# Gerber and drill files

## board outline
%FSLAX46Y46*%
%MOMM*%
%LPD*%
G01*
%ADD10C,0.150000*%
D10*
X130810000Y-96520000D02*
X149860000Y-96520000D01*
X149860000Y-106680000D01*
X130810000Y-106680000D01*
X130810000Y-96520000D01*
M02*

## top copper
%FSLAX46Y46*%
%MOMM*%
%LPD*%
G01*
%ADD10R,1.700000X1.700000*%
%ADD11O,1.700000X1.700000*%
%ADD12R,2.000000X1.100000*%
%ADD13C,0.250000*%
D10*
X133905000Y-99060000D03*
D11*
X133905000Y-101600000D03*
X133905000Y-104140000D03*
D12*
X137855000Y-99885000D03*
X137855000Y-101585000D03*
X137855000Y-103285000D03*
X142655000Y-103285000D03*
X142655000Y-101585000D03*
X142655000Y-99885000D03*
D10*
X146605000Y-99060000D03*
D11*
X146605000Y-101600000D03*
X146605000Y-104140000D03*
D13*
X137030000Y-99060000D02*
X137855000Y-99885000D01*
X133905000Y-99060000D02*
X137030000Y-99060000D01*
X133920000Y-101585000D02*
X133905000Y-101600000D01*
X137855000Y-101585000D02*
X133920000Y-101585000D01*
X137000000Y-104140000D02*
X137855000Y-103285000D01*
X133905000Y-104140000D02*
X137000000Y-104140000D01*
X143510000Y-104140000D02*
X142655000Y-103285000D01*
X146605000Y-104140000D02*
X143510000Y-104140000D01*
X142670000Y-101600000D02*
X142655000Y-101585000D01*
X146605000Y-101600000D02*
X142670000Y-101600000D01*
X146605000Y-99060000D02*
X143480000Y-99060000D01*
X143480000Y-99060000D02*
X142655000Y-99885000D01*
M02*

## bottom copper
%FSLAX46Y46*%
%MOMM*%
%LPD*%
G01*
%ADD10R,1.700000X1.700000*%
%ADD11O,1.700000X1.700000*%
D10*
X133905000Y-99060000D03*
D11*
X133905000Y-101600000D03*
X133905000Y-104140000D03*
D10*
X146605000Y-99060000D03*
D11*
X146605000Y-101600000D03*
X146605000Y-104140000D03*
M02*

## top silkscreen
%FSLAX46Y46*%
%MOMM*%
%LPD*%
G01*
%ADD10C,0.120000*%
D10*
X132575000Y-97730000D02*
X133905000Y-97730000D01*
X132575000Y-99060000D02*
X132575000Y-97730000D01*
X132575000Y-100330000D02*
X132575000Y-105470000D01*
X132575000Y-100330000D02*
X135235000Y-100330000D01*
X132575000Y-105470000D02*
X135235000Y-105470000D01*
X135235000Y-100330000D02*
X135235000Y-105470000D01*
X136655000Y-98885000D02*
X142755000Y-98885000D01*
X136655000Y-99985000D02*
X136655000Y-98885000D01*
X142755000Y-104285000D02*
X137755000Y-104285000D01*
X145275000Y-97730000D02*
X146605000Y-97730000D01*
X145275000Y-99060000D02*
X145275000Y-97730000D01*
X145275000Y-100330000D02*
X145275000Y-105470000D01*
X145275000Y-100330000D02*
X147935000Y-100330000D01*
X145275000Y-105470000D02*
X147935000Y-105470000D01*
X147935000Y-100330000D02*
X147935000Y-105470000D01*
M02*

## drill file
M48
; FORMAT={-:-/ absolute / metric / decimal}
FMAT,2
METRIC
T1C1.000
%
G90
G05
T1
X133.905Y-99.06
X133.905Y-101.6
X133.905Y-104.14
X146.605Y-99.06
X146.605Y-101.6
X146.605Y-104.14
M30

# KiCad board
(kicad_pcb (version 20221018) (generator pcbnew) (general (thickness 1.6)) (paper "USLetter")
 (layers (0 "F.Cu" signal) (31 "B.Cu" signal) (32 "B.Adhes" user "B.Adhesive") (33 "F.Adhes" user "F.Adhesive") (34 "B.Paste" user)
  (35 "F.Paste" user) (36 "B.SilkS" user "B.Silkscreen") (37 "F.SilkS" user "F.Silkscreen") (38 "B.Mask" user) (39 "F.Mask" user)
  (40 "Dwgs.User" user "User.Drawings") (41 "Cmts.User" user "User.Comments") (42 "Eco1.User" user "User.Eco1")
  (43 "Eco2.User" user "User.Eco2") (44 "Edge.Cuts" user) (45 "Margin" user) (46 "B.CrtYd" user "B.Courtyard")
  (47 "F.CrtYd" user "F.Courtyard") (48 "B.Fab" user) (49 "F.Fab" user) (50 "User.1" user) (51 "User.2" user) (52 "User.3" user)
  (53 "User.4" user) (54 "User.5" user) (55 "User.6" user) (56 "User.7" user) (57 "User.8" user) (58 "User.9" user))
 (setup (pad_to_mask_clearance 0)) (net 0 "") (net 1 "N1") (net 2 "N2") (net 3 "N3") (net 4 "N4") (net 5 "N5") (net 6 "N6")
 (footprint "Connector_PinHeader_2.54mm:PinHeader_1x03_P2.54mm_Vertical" (layer "F.Cu") (at 133.905 99.06)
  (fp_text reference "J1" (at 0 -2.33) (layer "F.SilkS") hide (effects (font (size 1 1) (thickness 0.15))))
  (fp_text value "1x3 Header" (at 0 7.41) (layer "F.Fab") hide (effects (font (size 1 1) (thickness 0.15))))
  (fp_line (start -1.33 -1.33) (end 0 -1.33) (stroke (width 0.12) (type solid)) (layer "F.SilkS"))
  (fp_line (start -1.33 0) (end -1.33 -1.33) (stroke (width 0.12) (type solid)) (layer "F.SilkS"))
  (fp_line (start -1.33 1.27) (end -1.33 6.41) (stroke (width 0.12) (type solid)) (layer "F.SilkS"))
  (fp_line (start -1.33 1.27) (end 1.33 1.27) (stroke (width 0.12) (type solid)) (layer "F.SilkS"))
  (fp_line (start -1.33 6.41) (end 1.33 6.41) (stroke (width 0.12) (type solid)) (layer "F.SilkS"))
  (fp_line (start 1.33 1.27) (end 1.33 6.41) (stroke (width 0.12) (type solid)) (layer "F.SilkS"))
  (pad "1" thru_hole rect (at 0 0) (size 1.7 1.7) (drill 1) (layers "*.Cu" "*.Mask") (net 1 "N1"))
  (pad "2" thru_hole oval (at 0 2.54) (size 1.7 1.7) (drill 1) (layers "*.Cu" "*.Mask") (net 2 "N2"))
  (pad "3" thru_hole oval (at 0 5.08) (size 1.7 1.7) (drill 1) (layers "*.Cu" "*.Mask") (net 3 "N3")))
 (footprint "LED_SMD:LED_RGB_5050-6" (layer "F.Cu") (at 140.255 101.585)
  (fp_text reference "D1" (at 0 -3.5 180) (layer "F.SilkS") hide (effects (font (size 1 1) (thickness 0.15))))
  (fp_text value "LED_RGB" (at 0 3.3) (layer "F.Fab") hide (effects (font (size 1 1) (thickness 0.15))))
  (fp_line (start -3.6 -2.7) (end 2.5 -2.7) (stroke (width 0.12) (type solid)) (layer "F.SilkS"))
  (fp_line (start -3.6 -1.6) (end -3.6 -2.7) (stroke (width 0.12) (type solid)) (layer "F.SilkS"))
  (fp_line (start 2.5 2.7) (end -2.5 2.7) (stroke (width 0.12) (type solid)) (layer "F.SilkS"))
  (pad "1" smd rect (at -2.4 -1.7 90) (size 1.1 2) (layers "F.Cu" "F.Paste" "F.Mask") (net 1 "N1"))
  (pad "2" smd rect (at -2.4 0 90) (size 1.1 2) (layers "F.Cu" "F.Paste" "F.Mask") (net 2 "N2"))
  (pad "3" smd rect (at -2.4 1.7 90) (size 1.1 2) (layers "F.Cu" "F.Paste" "F.Mask") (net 3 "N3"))
  (pad "4" smd rect (at 2.4 1.7 90) (size 1.1 2) (layers "F.Cu" "F.Paste" "F.Mask") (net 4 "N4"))
  (pad "5" smd rect (at 2.4 0 90) (size 1.1 2) (layers "F.Cu" "F.Paste" "F.Mask") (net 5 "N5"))
  (pad "6" smd rect (at 2.4 -1.7 90) (size 1.1 2) (layers "F.Cu" "F.Paste" "F.Mask") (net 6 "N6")))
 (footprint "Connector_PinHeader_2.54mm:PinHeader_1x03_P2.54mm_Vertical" (layer "F.Cu") (at 146.605 99.06)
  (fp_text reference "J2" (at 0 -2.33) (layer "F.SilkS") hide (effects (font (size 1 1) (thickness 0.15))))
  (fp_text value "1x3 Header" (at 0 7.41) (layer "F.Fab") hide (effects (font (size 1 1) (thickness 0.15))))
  (fp_line (start -1.33 -1.33) (end 0 -1.33) (stroke (width 0.12) (type solid)) (layer "F.SilkS"))
  (fp_line (start -1.33 0) (end -1.33 -1.33) (stroke (width 0.12) (type solid)) (layer "F.SilkS"))
  (fp_line (start -1.33 1.27) (end -1.33 6.41) (stroke (width 0.12) (type solid)) (layer "F.SilkS"))
  (fp_line (start -1.33 1.27) (end 1.33 1.27) (stroke (width 0.12) (type solid)) (layer "F.SilkS"))
  (fp_line (start -1.33 6.41) (end 1.33 6.41) (stroke (width 0.12) (type solid)) (layer "F.SilkS"))
  (fp_line (start 1.33 1.27) (end 1.33 6.41) (stroke (width 0.12) (type solid)) (layer "F.SilkS"))
  (pad "1" thru_hole rect (at 0 0) (size 1.7 1.7) (drill 1) (layers "*.Cu" "*.Mask") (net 6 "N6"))
  (pad "2" thru_hole oval (at 0 2.54) (size 1.7 1.7) (drill 1) (layers "*.Cu" "*.Mask") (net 5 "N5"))
  (pad "3" thru_hole oval (at 0 5.08) (size 1.7 1.7) (drill 1) (layers "*.Cu" "*.Mask") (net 4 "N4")))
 (gr_rect (start 130.81 96.52) (end 149.86 106.68) (stroke (width 0.15) (type solid)) (fill none) (layer "Edge.Cuts"))
 (segment (start 137.03 99.06) (end 137.855 99.885) (width 0.25) (layer "F.Cu") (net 1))
 (segment (start 133.905 99.06) (end 137.03 99.06) (width 0.25) (layer "F.Cu") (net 1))
 (segment (start 133.92 101.585) (end 133.905 101.6) (width 0.25) (layer "F.Cu") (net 2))
 (segment (start 137.855 101.585) (end 133.92 101.585) (width 0.25) (layer "F.Cu") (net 2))
 (segment (start 137 104.14) (end 137.855 103.285) (width 0.25) (layer "F.Cu") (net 3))
 (segment (start 133.905 104.14) (end 137 104.14) (width 0.25) (layer "F.Cu") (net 3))
 (segment (start 143.51 104.14) (end 142.655 103.285) (width 0.25) (layer "F.Cu") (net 4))
 (segment (start 146.605 104.14) (end 143.51 104.14) (width 0.25) (layer "F.Cu") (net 4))
 (segment (start 142.67 101.6) (end 142.655 101.585) (width 0.25) (layer "F.Cu") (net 5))
 (segment (start 146.605 101.6) (end 142.67 101.6) (width 0.25) (layer "F.Cu") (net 5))
 (segment (start 146.605 99.06) (end 143.48 99.06) (width 0.25) (layer "F.Cu") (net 6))
 (segment (start 143.48 99.06) (end 142.655 99.885) (width 0.25) (layer "F.Cu") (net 6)))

